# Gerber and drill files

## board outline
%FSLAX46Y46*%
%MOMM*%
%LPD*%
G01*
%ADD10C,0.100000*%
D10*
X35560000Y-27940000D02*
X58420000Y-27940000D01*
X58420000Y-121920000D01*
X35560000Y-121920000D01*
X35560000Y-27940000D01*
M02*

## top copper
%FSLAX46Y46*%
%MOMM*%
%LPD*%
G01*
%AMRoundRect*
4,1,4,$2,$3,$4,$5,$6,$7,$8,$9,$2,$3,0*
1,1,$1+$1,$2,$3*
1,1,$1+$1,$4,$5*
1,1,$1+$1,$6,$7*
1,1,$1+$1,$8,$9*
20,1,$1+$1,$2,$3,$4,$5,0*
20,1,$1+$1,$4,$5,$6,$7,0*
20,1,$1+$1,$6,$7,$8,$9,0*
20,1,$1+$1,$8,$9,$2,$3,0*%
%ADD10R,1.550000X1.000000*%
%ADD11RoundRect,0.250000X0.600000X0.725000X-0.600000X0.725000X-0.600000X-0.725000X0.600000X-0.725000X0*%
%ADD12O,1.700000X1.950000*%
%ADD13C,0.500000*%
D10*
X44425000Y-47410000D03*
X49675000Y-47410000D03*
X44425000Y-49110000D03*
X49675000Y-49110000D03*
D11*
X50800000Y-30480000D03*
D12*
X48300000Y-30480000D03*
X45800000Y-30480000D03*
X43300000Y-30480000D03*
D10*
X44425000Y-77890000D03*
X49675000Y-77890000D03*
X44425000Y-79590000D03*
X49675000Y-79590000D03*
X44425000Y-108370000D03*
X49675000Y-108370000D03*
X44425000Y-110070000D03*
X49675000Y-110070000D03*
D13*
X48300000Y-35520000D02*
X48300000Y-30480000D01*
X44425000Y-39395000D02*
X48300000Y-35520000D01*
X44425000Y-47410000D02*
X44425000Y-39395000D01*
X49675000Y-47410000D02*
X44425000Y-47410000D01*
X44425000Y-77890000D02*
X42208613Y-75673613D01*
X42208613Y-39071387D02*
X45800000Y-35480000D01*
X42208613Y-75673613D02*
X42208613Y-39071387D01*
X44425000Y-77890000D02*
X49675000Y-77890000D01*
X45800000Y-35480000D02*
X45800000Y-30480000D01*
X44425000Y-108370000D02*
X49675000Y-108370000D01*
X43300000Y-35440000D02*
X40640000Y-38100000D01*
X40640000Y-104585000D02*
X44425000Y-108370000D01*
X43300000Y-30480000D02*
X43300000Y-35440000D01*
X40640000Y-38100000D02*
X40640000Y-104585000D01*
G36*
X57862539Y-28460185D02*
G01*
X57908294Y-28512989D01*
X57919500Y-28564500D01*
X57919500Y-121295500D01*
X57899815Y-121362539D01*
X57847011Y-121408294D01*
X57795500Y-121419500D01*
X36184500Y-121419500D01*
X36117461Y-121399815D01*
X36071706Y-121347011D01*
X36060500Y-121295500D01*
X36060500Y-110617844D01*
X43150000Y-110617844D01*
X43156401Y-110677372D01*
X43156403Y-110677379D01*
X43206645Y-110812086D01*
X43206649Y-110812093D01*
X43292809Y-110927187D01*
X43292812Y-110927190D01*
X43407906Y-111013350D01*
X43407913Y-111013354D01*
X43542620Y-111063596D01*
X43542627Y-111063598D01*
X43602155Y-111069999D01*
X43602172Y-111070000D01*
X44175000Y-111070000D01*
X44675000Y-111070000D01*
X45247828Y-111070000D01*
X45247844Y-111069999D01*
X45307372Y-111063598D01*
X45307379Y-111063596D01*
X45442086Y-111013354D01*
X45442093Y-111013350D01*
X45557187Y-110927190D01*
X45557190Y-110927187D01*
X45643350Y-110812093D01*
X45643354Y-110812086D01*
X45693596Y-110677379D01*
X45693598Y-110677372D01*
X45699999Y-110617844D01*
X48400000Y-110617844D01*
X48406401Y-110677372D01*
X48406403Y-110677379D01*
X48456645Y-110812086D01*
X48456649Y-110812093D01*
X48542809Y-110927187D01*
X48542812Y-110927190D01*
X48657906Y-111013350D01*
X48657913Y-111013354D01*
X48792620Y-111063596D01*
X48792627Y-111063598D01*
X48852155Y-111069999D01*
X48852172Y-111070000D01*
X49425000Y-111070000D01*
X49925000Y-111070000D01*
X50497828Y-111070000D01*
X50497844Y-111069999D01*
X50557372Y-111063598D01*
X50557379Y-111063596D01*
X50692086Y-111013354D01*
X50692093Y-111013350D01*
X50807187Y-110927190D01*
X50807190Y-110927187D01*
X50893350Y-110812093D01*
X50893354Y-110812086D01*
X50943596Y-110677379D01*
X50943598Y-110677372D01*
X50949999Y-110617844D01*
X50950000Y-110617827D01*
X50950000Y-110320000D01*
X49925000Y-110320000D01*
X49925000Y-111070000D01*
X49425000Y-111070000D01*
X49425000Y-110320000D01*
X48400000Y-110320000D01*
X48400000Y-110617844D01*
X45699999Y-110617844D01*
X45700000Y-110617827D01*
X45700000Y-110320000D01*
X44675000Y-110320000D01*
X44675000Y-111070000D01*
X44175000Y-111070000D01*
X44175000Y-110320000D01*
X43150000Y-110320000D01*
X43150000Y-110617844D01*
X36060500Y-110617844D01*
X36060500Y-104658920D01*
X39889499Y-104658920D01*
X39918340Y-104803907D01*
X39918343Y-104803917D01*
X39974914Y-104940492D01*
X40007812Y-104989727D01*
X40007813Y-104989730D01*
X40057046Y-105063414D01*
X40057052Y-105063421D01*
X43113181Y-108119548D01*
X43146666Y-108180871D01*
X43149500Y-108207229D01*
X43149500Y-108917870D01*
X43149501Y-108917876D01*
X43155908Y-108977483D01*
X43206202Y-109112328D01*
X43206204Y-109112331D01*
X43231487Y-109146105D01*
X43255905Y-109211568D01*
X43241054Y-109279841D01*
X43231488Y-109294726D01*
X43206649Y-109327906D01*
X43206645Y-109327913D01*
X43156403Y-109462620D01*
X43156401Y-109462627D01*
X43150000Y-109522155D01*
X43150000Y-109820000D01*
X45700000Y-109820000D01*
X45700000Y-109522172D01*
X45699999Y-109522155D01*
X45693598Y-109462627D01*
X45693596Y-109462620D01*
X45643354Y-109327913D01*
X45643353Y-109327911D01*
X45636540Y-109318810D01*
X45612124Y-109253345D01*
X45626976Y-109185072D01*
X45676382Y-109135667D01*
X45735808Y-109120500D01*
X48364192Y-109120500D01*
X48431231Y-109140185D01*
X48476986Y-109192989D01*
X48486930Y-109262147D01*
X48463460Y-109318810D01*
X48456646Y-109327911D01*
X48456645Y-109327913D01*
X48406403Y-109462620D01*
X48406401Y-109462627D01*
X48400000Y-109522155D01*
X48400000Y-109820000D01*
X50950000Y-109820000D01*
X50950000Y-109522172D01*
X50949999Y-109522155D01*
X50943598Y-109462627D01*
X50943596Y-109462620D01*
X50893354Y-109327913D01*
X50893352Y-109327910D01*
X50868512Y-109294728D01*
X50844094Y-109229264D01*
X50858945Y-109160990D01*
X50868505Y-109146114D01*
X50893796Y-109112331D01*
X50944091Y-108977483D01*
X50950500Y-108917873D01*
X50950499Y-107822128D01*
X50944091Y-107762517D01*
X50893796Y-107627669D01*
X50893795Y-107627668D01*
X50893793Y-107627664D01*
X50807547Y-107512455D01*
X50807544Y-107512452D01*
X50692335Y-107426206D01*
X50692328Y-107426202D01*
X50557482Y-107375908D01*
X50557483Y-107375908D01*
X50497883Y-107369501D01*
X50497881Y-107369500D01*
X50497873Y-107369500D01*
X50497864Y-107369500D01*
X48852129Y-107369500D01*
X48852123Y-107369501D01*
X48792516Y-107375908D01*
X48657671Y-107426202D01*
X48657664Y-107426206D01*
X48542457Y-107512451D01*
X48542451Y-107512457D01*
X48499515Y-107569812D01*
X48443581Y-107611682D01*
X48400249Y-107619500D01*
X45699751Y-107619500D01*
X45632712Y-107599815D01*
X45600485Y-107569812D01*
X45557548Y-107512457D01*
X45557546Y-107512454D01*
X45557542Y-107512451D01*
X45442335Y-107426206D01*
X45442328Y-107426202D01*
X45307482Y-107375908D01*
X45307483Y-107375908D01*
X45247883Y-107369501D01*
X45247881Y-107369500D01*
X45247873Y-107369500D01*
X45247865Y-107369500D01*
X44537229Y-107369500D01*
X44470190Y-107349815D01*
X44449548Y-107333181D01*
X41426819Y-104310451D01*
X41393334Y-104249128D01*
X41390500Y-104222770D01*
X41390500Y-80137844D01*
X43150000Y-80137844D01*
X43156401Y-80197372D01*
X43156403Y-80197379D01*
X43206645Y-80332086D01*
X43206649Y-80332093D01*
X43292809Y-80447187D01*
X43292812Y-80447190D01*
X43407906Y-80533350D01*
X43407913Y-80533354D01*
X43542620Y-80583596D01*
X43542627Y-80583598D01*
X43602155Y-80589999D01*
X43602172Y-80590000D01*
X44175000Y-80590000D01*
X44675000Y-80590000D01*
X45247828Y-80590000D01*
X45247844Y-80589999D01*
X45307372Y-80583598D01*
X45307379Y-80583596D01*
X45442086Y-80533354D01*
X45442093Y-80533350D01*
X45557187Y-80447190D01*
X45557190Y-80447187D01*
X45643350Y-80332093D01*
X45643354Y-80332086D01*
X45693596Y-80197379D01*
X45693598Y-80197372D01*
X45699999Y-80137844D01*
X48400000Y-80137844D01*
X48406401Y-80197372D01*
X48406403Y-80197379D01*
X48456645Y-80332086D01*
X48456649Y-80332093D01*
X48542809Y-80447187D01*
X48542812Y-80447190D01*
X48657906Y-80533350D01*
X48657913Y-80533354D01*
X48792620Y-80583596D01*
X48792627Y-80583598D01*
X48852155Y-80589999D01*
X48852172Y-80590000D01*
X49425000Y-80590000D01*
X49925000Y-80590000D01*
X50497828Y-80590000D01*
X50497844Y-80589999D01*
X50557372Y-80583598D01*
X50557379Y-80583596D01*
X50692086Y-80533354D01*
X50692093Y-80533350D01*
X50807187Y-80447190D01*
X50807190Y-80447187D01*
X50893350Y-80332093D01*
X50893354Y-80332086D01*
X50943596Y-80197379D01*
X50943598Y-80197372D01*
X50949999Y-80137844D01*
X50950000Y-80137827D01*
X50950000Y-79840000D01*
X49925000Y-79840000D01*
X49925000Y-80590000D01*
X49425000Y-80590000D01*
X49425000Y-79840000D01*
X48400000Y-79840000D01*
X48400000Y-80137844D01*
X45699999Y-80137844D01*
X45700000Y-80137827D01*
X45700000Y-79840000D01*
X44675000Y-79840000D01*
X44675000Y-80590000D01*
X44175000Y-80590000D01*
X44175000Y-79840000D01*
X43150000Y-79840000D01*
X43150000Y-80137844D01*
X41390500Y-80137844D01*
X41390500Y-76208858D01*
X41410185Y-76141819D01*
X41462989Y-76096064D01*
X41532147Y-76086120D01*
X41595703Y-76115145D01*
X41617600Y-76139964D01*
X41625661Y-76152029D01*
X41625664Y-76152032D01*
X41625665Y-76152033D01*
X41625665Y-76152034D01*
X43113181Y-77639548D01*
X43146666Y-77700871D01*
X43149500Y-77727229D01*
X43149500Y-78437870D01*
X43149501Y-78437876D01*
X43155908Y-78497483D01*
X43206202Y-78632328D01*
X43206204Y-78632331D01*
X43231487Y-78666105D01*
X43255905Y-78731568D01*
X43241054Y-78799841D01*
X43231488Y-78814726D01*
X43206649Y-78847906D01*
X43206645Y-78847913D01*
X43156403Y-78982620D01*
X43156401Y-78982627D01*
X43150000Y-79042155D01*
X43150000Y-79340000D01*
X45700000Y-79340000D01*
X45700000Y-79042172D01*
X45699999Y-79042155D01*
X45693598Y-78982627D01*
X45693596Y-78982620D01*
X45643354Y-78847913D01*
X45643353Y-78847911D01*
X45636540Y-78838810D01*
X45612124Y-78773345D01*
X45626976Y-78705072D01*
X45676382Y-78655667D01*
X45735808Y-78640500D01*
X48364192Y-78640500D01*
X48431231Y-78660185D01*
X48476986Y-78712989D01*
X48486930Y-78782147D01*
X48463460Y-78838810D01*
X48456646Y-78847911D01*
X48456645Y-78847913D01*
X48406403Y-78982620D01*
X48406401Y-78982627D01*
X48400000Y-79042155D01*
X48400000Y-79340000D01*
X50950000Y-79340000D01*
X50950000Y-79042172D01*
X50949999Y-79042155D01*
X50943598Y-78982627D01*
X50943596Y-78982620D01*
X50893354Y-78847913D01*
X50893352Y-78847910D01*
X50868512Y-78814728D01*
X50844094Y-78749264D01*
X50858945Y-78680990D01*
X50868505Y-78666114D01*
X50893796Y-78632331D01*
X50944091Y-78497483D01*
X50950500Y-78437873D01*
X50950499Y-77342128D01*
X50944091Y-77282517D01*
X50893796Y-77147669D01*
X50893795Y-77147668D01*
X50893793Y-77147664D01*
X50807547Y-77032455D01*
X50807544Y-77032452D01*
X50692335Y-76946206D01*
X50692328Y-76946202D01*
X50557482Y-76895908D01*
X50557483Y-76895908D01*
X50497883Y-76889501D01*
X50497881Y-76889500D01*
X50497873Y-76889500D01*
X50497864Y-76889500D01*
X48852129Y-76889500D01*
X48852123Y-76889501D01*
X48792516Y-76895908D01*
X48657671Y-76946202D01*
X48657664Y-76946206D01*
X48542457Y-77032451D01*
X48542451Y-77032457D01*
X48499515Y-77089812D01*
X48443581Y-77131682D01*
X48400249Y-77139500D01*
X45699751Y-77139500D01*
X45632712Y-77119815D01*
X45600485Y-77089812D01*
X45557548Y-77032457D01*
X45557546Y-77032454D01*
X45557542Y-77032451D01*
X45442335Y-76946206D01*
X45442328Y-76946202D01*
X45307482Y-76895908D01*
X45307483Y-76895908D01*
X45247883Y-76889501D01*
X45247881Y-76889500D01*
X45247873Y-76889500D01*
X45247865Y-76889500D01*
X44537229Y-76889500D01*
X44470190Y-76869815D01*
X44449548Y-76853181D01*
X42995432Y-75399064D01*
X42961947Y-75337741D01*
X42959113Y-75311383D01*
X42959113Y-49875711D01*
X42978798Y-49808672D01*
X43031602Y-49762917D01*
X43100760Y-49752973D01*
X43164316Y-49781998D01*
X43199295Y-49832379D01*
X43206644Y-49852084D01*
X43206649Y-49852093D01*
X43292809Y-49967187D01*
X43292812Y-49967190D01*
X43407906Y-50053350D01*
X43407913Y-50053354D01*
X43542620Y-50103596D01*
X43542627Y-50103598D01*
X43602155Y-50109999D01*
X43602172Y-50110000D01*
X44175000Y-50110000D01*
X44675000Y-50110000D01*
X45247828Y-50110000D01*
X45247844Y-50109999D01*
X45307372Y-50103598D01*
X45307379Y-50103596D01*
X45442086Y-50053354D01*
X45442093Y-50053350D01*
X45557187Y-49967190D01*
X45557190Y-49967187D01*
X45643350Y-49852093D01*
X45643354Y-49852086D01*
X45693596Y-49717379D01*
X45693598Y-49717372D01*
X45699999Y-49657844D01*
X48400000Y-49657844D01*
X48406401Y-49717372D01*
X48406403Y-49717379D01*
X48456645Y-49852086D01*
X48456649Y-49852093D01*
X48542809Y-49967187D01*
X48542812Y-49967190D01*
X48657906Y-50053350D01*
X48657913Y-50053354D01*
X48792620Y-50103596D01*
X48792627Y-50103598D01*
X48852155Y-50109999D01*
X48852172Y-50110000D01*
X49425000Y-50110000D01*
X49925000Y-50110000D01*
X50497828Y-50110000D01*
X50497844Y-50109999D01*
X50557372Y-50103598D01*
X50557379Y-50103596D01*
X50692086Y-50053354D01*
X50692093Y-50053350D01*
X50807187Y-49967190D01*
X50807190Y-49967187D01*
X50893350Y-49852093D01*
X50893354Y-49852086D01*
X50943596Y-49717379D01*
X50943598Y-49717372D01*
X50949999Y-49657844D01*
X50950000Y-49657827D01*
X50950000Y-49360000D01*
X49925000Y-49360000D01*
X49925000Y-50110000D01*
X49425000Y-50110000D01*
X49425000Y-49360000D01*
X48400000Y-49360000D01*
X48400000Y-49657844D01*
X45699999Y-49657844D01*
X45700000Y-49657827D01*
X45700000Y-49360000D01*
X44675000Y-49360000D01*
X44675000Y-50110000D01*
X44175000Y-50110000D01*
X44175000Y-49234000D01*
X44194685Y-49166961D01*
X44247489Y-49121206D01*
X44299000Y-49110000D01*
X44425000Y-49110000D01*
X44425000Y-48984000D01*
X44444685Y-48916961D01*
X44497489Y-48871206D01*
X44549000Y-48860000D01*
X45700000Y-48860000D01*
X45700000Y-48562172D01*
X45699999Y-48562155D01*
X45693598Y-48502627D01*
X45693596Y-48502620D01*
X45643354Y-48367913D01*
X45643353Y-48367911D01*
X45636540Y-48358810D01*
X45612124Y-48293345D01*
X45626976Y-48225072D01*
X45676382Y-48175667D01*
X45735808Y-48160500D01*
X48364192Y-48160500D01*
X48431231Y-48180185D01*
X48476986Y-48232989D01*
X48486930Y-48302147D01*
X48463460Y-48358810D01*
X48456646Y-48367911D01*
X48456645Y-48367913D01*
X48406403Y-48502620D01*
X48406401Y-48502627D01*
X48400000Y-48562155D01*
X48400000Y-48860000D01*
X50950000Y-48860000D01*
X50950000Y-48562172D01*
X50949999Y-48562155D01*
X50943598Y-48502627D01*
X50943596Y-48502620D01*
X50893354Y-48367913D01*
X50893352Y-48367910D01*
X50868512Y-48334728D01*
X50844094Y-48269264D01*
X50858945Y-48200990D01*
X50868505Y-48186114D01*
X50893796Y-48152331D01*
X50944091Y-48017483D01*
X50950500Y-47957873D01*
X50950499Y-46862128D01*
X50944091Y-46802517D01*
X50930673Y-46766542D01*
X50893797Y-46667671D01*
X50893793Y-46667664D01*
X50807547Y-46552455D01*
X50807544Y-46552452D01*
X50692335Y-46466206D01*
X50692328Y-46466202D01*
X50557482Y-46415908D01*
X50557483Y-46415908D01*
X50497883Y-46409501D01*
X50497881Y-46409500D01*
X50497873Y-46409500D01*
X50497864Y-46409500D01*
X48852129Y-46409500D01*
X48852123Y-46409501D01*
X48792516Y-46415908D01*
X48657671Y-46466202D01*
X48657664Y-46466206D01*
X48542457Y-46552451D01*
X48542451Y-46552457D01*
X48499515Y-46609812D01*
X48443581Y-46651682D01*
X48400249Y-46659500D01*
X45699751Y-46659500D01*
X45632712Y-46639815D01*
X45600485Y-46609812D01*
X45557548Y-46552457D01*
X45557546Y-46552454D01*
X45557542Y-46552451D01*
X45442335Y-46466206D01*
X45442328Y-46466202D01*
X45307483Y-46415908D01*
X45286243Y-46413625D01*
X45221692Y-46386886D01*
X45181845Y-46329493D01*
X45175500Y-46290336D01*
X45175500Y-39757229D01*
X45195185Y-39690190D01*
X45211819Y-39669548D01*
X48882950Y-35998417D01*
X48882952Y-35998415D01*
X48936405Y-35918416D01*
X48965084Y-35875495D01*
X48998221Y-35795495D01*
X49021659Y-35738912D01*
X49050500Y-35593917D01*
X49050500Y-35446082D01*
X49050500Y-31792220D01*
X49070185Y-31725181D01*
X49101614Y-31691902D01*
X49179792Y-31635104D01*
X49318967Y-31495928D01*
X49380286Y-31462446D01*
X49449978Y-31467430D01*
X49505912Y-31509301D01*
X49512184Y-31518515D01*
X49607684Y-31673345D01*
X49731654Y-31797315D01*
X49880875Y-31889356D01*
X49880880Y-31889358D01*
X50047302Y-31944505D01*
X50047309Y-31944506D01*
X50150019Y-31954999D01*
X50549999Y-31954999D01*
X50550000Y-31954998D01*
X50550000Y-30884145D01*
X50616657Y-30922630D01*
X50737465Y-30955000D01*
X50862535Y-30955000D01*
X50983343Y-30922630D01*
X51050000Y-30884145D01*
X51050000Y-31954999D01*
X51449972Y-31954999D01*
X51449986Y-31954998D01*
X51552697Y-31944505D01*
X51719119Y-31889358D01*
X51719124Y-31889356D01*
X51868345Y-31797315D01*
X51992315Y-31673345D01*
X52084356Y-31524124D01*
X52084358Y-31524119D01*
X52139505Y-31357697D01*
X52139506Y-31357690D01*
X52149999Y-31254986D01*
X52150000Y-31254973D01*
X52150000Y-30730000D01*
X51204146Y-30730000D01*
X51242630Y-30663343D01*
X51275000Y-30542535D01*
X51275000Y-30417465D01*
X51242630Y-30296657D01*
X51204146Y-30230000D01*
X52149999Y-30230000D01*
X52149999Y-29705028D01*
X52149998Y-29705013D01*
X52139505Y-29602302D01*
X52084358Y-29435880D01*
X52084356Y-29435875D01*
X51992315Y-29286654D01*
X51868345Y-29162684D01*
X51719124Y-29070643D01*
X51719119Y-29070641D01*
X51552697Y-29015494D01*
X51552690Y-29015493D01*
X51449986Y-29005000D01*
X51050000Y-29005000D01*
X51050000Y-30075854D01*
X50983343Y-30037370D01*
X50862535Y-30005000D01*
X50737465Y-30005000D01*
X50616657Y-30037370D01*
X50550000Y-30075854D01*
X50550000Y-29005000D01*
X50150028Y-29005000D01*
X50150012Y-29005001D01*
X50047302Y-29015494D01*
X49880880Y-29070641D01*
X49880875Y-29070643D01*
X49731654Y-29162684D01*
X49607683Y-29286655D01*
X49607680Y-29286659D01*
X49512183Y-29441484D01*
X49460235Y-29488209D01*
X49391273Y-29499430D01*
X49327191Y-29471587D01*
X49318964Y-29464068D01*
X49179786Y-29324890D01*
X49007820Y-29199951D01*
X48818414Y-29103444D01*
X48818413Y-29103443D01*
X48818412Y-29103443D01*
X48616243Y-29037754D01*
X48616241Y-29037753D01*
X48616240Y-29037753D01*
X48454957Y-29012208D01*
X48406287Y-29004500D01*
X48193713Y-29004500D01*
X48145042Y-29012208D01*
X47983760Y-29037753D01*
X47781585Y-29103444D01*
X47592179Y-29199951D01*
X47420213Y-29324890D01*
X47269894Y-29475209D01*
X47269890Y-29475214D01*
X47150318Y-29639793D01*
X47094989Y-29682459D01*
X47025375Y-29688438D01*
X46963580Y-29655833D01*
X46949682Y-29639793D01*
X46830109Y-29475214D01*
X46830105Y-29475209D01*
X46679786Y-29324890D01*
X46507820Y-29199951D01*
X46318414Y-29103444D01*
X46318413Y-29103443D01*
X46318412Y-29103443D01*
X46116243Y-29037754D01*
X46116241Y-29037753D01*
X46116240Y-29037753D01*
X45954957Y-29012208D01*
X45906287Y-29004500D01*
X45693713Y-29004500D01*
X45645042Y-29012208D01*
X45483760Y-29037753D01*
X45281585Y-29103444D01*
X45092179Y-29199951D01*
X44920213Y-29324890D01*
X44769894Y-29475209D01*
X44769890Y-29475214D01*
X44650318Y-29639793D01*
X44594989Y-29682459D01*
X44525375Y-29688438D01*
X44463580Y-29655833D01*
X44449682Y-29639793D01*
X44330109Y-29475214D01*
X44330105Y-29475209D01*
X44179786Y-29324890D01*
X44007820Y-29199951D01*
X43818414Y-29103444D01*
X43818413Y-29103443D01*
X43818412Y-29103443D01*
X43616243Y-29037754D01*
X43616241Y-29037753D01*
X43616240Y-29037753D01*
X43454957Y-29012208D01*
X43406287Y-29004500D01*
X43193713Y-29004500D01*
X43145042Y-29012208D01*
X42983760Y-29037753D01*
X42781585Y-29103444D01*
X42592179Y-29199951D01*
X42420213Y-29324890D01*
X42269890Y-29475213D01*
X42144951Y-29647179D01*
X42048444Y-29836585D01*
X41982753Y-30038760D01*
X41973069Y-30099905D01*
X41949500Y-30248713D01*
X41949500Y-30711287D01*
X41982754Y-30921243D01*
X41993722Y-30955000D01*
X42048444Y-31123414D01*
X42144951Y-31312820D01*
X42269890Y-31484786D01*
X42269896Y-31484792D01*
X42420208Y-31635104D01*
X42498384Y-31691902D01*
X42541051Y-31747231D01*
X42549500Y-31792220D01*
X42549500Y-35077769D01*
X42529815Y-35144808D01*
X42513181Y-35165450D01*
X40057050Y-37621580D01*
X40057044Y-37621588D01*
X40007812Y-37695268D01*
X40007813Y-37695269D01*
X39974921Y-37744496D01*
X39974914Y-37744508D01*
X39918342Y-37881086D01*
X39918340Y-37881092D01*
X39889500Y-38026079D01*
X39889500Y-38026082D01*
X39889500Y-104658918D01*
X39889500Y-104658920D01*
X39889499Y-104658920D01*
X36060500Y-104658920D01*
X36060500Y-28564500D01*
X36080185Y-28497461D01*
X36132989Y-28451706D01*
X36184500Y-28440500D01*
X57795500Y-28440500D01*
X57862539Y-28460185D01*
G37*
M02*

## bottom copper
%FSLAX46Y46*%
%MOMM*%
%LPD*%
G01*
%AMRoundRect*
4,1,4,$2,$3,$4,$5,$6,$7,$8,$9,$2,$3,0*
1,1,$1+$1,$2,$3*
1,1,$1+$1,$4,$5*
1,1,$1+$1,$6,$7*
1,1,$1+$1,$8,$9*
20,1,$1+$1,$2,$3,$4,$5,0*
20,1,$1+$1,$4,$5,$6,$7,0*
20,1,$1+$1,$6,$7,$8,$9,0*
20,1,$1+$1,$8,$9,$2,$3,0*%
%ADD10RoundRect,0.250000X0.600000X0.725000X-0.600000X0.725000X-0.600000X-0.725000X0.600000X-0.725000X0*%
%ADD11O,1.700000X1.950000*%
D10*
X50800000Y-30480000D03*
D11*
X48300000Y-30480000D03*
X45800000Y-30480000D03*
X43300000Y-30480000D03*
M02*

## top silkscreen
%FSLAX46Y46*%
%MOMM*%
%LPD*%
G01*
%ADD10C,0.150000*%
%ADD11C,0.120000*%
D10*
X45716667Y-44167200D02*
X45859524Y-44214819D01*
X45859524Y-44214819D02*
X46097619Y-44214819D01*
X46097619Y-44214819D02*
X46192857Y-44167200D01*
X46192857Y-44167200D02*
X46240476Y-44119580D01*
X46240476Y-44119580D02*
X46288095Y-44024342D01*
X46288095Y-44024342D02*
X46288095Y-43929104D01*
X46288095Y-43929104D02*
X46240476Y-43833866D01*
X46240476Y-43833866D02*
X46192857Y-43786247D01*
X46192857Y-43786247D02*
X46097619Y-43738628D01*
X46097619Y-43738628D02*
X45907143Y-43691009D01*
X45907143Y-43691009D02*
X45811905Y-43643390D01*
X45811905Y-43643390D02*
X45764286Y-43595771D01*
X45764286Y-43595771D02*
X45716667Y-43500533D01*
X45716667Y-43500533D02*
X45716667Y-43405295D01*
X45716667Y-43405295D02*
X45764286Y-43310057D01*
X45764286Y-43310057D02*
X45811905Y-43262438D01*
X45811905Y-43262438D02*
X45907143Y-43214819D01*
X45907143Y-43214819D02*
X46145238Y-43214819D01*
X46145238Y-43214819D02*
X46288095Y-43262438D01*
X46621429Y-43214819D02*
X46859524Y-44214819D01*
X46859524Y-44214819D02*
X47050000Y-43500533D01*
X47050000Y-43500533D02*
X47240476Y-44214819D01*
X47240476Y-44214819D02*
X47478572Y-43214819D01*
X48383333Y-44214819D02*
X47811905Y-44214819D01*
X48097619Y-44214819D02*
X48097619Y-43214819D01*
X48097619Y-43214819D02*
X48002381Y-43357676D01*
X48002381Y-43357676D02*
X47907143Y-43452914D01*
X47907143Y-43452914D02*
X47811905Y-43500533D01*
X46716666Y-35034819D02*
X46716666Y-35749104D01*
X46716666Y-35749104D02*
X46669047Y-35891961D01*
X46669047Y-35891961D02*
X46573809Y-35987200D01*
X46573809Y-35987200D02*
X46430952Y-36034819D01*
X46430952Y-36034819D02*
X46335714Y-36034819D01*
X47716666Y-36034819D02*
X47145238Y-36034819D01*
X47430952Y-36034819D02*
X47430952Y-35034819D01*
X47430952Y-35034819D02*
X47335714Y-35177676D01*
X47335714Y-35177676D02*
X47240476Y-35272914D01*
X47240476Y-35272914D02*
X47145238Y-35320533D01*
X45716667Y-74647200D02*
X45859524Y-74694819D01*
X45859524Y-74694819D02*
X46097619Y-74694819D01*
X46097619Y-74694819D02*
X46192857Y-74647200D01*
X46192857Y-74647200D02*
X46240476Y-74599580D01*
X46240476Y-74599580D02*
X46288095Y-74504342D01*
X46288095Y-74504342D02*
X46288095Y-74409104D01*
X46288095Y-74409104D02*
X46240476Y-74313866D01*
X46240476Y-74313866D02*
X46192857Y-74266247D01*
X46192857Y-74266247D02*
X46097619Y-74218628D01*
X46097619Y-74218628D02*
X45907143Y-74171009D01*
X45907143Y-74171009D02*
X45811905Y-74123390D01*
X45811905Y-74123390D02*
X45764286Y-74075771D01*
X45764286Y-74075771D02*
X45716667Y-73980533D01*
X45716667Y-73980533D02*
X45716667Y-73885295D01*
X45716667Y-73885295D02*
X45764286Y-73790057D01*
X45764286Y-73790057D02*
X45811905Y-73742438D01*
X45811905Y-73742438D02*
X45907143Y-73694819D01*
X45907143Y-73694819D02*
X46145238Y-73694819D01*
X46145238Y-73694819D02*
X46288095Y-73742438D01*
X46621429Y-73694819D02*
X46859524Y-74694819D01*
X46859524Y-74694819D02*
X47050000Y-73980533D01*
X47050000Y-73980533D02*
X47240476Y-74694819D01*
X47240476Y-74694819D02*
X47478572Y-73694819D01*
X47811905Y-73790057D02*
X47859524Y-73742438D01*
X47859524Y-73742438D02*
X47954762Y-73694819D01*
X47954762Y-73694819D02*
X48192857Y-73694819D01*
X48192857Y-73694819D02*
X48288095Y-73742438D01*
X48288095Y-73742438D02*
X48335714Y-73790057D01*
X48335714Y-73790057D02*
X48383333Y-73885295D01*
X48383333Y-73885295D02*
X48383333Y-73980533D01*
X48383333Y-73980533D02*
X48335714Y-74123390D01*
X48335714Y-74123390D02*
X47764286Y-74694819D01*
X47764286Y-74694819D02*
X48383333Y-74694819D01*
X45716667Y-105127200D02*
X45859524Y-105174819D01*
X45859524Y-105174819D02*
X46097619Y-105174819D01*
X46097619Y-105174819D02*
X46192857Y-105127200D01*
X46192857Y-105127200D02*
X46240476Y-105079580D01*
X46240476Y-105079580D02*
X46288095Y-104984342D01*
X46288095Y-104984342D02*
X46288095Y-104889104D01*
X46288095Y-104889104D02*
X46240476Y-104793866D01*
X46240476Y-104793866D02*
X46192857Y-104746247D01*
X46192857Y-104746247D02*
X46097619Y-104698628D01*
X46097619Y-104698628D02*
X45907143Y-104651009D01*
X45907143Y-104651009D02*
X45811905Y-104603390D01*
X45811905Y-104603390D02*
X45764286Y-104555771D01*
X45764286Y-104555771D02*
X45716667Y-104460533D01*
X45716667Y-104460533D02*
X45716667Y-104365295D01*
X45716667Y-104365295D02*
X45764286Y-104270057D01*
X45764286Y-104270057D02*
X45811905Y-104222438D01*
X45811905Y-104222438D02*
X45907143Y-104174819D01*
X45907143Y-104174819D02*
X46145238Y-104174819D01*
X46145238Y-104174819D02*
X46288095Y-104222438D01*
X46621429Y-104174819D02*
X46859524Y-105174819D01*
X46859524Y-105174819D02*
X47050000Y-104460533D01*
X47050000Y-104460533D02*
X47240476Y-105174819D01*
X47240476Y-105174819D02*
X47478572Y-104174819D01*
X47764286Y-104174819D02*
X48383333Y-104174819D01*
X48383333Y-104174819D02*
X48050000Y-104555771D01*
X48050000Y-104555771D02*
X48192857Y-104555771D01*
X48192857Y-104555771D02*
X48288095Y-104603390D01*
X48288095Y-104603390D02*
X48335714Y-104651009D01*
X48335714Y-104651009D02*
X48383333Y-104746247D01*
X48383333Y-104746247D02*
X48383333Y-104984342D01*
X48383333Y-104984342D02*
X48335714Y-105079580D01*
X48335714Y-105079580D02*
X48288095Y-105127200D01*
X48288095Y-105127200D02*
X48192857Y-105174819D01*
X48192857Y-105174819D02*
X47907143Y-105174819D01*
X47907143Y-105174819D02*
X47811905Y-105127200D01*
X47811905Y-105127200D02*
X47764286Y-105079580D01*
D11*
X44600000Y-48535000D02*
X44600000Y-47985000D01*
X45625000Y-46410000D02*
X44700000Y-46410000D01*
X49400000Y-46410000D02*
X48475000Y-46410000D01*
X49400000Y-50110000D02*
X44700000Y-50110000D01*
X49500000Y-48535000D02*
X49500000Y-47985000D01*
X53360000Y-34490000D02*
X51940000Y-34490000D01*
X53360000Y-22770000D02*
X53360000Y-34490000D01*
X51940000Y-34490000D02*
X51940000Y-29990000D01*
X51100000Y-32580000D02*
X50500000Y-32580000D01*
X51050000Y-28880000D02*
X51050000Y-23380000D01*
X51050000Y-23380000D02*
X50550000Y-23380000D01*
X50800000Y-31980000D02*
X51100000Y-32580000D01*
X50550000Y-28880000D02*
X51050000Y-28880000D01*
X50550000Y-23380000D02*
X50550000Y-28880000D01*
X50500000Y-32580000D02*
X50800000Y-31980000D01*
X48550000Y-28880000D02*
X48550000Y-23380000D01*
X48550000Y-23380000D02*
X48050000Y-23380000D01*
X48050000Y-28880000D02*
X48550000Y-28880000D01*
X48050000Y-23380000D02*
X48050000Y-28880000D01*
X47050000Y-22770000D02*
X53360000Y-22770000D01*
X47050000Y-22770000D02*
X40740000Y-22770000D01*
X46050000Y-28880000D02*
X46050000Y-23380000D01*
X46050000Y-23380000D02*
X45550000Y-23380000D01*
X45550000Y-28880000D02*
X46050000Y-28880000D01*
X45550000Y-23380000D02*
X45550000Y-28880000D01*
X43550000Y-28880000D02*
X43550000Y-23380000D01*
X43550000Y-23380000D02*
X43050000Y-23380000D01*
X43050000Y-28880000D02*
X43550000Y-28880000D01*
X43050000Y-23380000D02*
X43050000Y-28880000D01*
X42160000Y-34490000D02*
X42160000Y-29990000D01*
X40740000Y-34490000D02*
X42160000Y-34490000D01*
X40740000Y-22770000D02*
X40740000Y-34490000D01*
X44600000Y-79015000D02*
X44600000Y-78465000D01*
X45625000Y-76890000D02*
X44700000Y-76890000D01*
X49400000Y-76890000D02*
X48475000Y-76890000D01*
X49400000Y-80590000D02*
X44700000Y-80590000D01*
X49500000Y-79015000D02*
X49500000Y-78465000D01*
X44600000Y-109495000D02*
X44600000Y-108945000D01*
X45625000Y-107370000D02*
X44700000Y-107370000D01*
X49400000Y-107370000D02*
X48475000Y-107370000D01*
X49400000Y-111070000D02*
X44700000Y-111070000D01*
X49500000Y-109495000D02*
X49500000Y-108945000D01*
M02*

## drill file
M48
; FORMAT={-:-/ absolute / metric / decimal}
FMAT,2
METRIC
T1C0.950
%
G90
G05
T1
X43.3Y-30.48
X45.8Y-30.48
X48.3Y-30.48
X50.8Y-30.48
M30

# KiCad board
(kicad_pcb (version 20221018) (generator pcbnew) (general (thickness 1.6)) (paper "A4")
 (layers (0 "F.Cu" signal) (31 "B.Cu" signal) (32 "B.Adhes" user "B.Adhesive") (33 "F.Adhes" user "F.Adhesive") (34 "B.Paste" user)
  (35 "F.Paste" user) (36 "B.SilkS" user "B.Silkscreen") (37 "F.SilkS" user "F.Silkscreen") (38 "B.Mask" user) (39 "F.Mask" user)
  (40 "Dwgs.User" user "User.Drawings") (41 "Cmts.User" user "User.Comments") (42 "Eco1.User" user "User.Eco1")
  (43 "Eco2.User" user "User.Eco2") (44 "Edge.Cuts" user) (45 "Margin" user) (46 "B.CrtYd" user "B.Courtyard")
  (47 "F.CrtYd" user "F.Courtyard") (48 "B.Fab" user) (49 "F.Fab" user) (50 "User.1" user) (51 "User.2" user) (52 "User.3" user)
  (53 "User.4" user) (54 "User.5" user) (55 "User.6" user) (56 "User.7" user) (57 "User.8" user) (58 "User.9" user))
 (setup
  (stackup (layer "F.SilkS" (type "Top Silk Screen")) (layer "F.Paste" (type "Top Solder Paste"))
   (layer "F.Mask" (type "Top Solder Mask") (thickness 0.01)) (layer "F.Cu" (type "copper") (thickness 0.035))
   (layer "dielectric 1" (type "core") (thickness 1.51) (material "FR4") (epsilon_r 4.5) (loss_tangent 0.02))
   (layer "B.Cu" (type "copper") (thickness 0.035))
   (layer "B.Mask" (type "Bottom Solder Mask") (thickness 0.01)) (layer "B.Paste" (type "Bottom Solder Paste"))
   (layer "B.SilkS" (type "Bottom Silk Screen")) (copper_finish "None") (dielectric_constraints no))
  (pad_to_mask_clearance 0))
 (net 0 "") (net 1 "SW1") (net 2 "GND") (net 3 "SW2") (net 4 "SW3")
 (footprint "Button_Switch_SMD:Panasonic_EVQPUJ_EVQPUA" (layer "F.Cu") (at 47.05 48.26)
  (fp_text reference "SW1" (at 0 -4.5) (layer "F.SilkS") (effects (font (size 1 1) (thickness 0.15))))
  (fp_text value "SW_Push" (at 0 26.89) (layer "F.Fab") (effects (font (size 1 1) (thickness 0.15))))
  (fp_line (start -2.45 0.275) (end -2.45 -0.275) (stroke (width 0.12) (type solid)) (layer "F.SilkS"))
  (fp_line (start -1.425 -1.85) (end -2.35 -1.85) (stroke (width 0.12) (type solid)) (layer "F.SilkS"))
  (fp_line (start 2.35 -1.85) (end 1.425 -1.85) (stroke (width 0.12) (type solid)) (layer "F.SilkS"))
  (fp_line (start 2.35 1.85) (end -2.35 1.85) (stroke (width 0.12) (type solid)) (layer "F.SilkS"))
  (fp_line (start 2.45 0.275) (end 2.45 -0.275) (stroke (width 0.12) (type solid)) (layer "F.SilkS"))
  (pad "1" smd rect (at -2.625 -0.85 180) (size 1.55 1) (layers "F.Cu" "F.Paste" "F.Mask") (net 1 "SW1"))
  (pad "1" smd rect (at 2.625 -0.85 180) (size 1.55 1) (layers "F.Cu" "F.Paste" "F.Mask") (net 1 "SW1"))
  (pad "2" smd rect (at -2.625 0.85 180) (size 1.55 1) (layers "F.Cu" "F.Paste" "F.Mask") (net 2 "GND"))
  (pad "2" smd rect (at 2.625 0.85 180) (size 1.55 1) (layers "F.Cu" "F.Paste" "F.Mask") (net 2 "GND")))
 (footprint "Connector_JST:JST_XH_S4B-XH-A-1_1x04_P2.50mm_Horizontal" (layer "F.Cu") (at 50.8 30.48 180)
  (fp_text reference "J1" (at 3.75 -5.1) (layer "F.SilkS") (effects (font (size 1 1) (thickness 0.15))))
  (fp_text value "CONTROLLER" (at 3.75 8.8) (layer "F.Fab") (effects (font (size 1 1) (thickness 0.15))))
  (fp_line (start -2.56 -4.01) (end -1.14 -4.01) (stroke (width 0.12) (type solid)) (layer "F.SilkS"))
  (fp_line (start -2.56 7.71) (end -2.56 -4.01) (stroke (width 0.12) (type solid)) (layer "F.SilkS"))
  (fp_line (start -1.14 -4.01) (end -1.14 0.49) (stroke (width 0.12) (type solid)) (layer "F.SilkS"))
  (fp_line (start -0.3 -2.1) (end 0.3 -2.1) (stroke (width 0.12) (type solid)) (layer "F.SilkS"))
  (fp_line (start -0.25 1.6) (end -0.25 7.1) (stroke (width 0.12) (type solid)) (layer "F.SilkS"))
  (fp_line (start -0.25 7.1) (end 0.25 7.1) (stroke (width 0.12) (type solid)) (layer "F.SilkS"))
  (fp_line (start 0 -1.5) (end -0.3 -2.1) (stroke (width 0.12) (type solid)) (layer "F.SilkS"))
  (fp_line (start 0.25 1.6) (end -0.25 1.6) (stroke (width 0.12) (type solid)) (layer "F.SilkS"))
  (fp_line (start 0.25 7.1) (end 0.25 1.6) (stroke (width 0.12) (type solid)) (layer "F.SilkS"))
  (fp_line (start 0.3 -2.1) (end 0 -1.5) (stroke (width 0.12) (type solid)) (layer "F.SilkS"))
  (fp_line (start 2.25 1.6) (end 2.25 7.1) (stroke (width 0.12) (type solid)) (layer "F.SilkS"))
  (fp_line (start 2.25 7.1) (end 2.75 7.1) (stroke (width 0.12) (type solid)) (layer "F.SilkS"))
  (fp_line (start 2.75 1.6) (end 2.25 1.6) (stroke (width 0.12) (type solid)) (layer "F.SilkS"))
  (fp_line (start 2.75 7.1) (end 2.75 1.6) (stroke (width 0.12) (type solid)) (layer "F.SilkS"))
  (fp_line (start 3.75 7.71) (end -2.56 7.71) (stroke (width 0.12) (type solid)) (layer "F.SilkS"))
  (fp_line (start 3.75 7.71) (end 10.06 7.71) (stroke (width 0.12) (type solid)) (layer "F.SilkS"))
  (fp_line (start 4.75 1.6) (end 4.75 7.1) (stroke (width 0.12) (type solid)) (layer "F.SilkS"))
  (fp_line (start 4.75 7.1) (end 5.25 7.1) (stroke (width 0.12) (type solid)) (layer "F.SilkS"))
  (fp_line (start 5.25 1.6) (end 4.75 1.6) (stroke (width 0.12) (type solid)) (layer "F.SilkS"))
  (fp_line (start 5.25 7.1) (end 5.25 1.6) (stroke (width 0.12) (type solid)) (layer "F.SilkS"))
  (fp_line (start 7.25 1.6) (end 7.25 7.1) (stroke (width 0.12) (type solid)) (layer "F.SilkS"))
  (fp_line (start 7.25 7.1) (end 7.75 7.1) (stroke (width 0.12) (type solid)) (layer "F.SilkS"))
  (fp_line (start 7.75 1.6) (end 7.25 1.6) (stroke (width 0.12) (type solid)) (layer "F.SilkS"))
  (fp_line (start 7.75 7.1) (end 7.75 1.6) (stroke (width 0.12) (type solid)) (layer "F.SilkS"))
  (fp_line (start 8.64 -4.01) (end 8.64 0.49) (stroke (width 0.12) (type solid)) (layer "F.SilkS"))
  (fp_line (start 10.06 -4.01) (end 8.64 -4.01) (stroke (width 0.12) (type solid)) (layer "F.SilkS"))
  (fp_line (start 10.06 7.71) (end 10.06 -4.01) (stroke (width 0.12) (type solid)) (layer "F.SilkS"))
  (pad "1" thru_hole roundrect (at 0 0 180) (size 1.7 1.95) (drill 0.95) (layers "*.Cu" "*.Mask") (roundrect_rratio 0.147059) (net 2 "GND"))
  (pad "2" thru_hole oval (at 2.5 0 180) (size 1.7 1.95) (drill 0.95) (layers "*.Cu" "*.Mask") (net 1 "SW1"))
  (pad "3" thru_hole oval (at 5 0 180) (size 1.7 1.95) (drill 0.95) (layers "*.Cu" "*.Mask") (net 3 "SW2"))
  (pad "4" thru_hole oval (at 7.5 0 180) (size 1.7 1.95) (drill 0.95) (layers "*.Cu" "*.Mask") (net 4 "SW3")))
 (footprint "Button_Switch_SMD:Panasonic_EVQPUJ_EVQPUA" (layer "F.Cu") (at 47.05 78.74)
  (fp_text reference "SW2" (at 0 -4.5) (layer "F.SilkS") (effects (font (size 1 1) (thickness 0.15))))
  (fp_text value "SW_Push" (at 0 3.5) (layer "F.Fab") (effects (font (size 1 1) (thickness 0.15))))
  (fp_line (start -2.45 0.275) (end -2.45 -0.275) (stroke (width 0.12) (type solid)) (layer "F.SilkS"))
  (fp_line (start -1.425 -1.85) (end -2.35 -1.85) (stroke (width 0.12) (type solid)) (layer "F.SilkS"))
  (fp_line (start 2.35 -1.85) (end 1.425 -1.85) (stroke (width 0.12) (type solid)) (layer "F.SilkS"))
  (fp_line (start 2.35 1.85) (end -2.35 1.85) (stroke (width 0.12) (type solid)) (layer "F.SilkS"))
  (fp_line (start 2.45 0.275) (end 2.45 -0.275) (stroke (width 0.12) (type solid)) (layer "F.SilkS"))
  (pad "1" smd rect (at -2.625 -0.85 180) (size 1.55 1) (layers "F.Cu" "F.Paste" "F.Mask") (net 3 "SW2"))
  (pad "1" smd rect (at 2.625 -0.85 180) (size 1.55 1) (layers "F.Cu" "F.Paste" "F.Mask") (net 3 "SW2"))
  (pad "2" smd rect (at -2.625 0.85 180) (size 1.55 1) (layers "F.Cu" "F.Paste" "F.Mask") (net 2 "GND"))
  (pad "2" smd rect (at 2.625 0.85 180) (size 1.55 1) (layers "F.Cu" "F.Paste" "F.Mask") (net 2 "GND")))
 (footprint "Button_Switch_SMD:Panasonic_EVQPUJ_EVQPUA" (layer "F.Cu") (at 47.05 109.22)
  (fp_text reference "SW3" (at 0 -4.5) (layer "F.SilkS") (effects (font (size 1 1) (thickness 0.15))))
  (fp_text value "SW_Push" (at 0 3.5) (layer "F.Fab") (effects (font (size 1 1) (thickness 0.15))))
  (fp_line (start -2.45 0.275) (end -2.45 -0.275) (stroke (width 0.12) (type solid)) (layer "F.SilkS"))
  (fp_line (start -1.425 -1.85) (end -2.35 -1.85) (stroke (width 0.12) (type solid)) (layer "F.SilkS"))
  (fp_line (start 2.35 -1.85) (end 1.425 -1.85) (stroke (width 0.12) (type solid)) (layer "F.SilkS"))
  (fp_line (start 2.35 1.85) (end -2.35 1.85) (stroke (width 0.12) (type solid)) (layer "F.SilkS"))
  (fp_line (start 2.45 0.275) (end 2.45 -0.275) (stroke (width 0.12) (type solid)) (layer "F.SilkS"))
  (pad "1" smd rect (at -2.625 -0.85 180) (size 1.55 1) (layers "F.Cu" "F.Paste" "F.Mask") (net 4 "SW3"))
  (pad "1" smd rect (at 2.625 -0.85 180) (size 1.55 1) (layers "F.Cu" "F.Paste" "F.Mask") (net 4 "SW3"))
  (pad "2" smd rect (at -2.625 0.85 180) (size 1.55 1) (layers "F.Cu" "F.Paste" "F.Mask") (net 2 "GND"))
  (pad "2" smd rect (at 2.625 0.85 180) (size 1.55 1) (layers "F.Cu" "F.Paste" "F.Mask") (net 2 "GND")))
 (gr_rect (start 35.56 27.94) (end 58.42 121.92) (stroke (width 0.1) (type default)) (fill none) (layer "Edge.Cuts"))
 (segment (start 48.3 35.52) (end 48.3 30.48) (width 0.5) (layer "F.Cu") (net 1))
 (segment (start 44.425 39.395) (end 48.3 35.52) (width 0.5) (layer "F.Cu") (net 1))
 (segment (start 44.425 47.41) (end 44.425 39.395) (width 0.5) (layer "F.Cu") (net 1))
 (segment (start 49.675 47.41) (end 44.425 47.41) (width 0.5) (layer "F.Cu") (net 1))
 (segment (start 44.425 77.89) (end 42.208613 75.673613) (width 0.5) (layer "F.Cu") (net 3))
 (segment (start 42.208613 39.071387) (end 45.8 35.48) (width 0.5) (layer "F.Cu") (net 3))
 (segment (start 42.208613 75.673613) (end 42.208613 39.071387) (width 0.5) (layer "F.Cu") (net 3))
 (segment (start 44.425 77.89) (end 49.675 77.89) (width 0.5) (layer "F.Cu") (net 3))
 (segment (start 45.8 35.48) (end 45.8 30.48) (width 0.5) (layer "F.Cu") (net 3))
 (segment (start 44.425 108.37) (end 49.675 108.37) (width 0.5) (layer "F.Cu") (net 4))
 (segment (start 43.3 35.44) (end 40.64 38.1) (width 0.5) (layer "F.Cu") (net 4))
 (segment (start 40.64 104.585) (end 44.425 108.37) (width 0.5) (layer "F.Cu") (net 4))
 (segment (start 43.3 30.48) (end 43.3 35.44) (width 0.5) (layer "F.Cu") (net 4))
 (segment (start 40.64 38.1) (end 40.64 104.585) (width 0.5) (layer "F.Cu") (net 4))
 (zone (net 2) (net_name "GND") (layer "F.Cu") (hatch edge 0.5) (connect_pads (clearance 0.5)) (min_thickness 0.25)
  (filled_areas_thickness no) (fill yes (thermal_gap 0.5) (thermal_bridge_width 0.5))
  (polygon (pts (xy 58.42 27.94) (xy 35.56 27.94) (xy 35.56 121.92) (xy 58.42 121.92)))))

